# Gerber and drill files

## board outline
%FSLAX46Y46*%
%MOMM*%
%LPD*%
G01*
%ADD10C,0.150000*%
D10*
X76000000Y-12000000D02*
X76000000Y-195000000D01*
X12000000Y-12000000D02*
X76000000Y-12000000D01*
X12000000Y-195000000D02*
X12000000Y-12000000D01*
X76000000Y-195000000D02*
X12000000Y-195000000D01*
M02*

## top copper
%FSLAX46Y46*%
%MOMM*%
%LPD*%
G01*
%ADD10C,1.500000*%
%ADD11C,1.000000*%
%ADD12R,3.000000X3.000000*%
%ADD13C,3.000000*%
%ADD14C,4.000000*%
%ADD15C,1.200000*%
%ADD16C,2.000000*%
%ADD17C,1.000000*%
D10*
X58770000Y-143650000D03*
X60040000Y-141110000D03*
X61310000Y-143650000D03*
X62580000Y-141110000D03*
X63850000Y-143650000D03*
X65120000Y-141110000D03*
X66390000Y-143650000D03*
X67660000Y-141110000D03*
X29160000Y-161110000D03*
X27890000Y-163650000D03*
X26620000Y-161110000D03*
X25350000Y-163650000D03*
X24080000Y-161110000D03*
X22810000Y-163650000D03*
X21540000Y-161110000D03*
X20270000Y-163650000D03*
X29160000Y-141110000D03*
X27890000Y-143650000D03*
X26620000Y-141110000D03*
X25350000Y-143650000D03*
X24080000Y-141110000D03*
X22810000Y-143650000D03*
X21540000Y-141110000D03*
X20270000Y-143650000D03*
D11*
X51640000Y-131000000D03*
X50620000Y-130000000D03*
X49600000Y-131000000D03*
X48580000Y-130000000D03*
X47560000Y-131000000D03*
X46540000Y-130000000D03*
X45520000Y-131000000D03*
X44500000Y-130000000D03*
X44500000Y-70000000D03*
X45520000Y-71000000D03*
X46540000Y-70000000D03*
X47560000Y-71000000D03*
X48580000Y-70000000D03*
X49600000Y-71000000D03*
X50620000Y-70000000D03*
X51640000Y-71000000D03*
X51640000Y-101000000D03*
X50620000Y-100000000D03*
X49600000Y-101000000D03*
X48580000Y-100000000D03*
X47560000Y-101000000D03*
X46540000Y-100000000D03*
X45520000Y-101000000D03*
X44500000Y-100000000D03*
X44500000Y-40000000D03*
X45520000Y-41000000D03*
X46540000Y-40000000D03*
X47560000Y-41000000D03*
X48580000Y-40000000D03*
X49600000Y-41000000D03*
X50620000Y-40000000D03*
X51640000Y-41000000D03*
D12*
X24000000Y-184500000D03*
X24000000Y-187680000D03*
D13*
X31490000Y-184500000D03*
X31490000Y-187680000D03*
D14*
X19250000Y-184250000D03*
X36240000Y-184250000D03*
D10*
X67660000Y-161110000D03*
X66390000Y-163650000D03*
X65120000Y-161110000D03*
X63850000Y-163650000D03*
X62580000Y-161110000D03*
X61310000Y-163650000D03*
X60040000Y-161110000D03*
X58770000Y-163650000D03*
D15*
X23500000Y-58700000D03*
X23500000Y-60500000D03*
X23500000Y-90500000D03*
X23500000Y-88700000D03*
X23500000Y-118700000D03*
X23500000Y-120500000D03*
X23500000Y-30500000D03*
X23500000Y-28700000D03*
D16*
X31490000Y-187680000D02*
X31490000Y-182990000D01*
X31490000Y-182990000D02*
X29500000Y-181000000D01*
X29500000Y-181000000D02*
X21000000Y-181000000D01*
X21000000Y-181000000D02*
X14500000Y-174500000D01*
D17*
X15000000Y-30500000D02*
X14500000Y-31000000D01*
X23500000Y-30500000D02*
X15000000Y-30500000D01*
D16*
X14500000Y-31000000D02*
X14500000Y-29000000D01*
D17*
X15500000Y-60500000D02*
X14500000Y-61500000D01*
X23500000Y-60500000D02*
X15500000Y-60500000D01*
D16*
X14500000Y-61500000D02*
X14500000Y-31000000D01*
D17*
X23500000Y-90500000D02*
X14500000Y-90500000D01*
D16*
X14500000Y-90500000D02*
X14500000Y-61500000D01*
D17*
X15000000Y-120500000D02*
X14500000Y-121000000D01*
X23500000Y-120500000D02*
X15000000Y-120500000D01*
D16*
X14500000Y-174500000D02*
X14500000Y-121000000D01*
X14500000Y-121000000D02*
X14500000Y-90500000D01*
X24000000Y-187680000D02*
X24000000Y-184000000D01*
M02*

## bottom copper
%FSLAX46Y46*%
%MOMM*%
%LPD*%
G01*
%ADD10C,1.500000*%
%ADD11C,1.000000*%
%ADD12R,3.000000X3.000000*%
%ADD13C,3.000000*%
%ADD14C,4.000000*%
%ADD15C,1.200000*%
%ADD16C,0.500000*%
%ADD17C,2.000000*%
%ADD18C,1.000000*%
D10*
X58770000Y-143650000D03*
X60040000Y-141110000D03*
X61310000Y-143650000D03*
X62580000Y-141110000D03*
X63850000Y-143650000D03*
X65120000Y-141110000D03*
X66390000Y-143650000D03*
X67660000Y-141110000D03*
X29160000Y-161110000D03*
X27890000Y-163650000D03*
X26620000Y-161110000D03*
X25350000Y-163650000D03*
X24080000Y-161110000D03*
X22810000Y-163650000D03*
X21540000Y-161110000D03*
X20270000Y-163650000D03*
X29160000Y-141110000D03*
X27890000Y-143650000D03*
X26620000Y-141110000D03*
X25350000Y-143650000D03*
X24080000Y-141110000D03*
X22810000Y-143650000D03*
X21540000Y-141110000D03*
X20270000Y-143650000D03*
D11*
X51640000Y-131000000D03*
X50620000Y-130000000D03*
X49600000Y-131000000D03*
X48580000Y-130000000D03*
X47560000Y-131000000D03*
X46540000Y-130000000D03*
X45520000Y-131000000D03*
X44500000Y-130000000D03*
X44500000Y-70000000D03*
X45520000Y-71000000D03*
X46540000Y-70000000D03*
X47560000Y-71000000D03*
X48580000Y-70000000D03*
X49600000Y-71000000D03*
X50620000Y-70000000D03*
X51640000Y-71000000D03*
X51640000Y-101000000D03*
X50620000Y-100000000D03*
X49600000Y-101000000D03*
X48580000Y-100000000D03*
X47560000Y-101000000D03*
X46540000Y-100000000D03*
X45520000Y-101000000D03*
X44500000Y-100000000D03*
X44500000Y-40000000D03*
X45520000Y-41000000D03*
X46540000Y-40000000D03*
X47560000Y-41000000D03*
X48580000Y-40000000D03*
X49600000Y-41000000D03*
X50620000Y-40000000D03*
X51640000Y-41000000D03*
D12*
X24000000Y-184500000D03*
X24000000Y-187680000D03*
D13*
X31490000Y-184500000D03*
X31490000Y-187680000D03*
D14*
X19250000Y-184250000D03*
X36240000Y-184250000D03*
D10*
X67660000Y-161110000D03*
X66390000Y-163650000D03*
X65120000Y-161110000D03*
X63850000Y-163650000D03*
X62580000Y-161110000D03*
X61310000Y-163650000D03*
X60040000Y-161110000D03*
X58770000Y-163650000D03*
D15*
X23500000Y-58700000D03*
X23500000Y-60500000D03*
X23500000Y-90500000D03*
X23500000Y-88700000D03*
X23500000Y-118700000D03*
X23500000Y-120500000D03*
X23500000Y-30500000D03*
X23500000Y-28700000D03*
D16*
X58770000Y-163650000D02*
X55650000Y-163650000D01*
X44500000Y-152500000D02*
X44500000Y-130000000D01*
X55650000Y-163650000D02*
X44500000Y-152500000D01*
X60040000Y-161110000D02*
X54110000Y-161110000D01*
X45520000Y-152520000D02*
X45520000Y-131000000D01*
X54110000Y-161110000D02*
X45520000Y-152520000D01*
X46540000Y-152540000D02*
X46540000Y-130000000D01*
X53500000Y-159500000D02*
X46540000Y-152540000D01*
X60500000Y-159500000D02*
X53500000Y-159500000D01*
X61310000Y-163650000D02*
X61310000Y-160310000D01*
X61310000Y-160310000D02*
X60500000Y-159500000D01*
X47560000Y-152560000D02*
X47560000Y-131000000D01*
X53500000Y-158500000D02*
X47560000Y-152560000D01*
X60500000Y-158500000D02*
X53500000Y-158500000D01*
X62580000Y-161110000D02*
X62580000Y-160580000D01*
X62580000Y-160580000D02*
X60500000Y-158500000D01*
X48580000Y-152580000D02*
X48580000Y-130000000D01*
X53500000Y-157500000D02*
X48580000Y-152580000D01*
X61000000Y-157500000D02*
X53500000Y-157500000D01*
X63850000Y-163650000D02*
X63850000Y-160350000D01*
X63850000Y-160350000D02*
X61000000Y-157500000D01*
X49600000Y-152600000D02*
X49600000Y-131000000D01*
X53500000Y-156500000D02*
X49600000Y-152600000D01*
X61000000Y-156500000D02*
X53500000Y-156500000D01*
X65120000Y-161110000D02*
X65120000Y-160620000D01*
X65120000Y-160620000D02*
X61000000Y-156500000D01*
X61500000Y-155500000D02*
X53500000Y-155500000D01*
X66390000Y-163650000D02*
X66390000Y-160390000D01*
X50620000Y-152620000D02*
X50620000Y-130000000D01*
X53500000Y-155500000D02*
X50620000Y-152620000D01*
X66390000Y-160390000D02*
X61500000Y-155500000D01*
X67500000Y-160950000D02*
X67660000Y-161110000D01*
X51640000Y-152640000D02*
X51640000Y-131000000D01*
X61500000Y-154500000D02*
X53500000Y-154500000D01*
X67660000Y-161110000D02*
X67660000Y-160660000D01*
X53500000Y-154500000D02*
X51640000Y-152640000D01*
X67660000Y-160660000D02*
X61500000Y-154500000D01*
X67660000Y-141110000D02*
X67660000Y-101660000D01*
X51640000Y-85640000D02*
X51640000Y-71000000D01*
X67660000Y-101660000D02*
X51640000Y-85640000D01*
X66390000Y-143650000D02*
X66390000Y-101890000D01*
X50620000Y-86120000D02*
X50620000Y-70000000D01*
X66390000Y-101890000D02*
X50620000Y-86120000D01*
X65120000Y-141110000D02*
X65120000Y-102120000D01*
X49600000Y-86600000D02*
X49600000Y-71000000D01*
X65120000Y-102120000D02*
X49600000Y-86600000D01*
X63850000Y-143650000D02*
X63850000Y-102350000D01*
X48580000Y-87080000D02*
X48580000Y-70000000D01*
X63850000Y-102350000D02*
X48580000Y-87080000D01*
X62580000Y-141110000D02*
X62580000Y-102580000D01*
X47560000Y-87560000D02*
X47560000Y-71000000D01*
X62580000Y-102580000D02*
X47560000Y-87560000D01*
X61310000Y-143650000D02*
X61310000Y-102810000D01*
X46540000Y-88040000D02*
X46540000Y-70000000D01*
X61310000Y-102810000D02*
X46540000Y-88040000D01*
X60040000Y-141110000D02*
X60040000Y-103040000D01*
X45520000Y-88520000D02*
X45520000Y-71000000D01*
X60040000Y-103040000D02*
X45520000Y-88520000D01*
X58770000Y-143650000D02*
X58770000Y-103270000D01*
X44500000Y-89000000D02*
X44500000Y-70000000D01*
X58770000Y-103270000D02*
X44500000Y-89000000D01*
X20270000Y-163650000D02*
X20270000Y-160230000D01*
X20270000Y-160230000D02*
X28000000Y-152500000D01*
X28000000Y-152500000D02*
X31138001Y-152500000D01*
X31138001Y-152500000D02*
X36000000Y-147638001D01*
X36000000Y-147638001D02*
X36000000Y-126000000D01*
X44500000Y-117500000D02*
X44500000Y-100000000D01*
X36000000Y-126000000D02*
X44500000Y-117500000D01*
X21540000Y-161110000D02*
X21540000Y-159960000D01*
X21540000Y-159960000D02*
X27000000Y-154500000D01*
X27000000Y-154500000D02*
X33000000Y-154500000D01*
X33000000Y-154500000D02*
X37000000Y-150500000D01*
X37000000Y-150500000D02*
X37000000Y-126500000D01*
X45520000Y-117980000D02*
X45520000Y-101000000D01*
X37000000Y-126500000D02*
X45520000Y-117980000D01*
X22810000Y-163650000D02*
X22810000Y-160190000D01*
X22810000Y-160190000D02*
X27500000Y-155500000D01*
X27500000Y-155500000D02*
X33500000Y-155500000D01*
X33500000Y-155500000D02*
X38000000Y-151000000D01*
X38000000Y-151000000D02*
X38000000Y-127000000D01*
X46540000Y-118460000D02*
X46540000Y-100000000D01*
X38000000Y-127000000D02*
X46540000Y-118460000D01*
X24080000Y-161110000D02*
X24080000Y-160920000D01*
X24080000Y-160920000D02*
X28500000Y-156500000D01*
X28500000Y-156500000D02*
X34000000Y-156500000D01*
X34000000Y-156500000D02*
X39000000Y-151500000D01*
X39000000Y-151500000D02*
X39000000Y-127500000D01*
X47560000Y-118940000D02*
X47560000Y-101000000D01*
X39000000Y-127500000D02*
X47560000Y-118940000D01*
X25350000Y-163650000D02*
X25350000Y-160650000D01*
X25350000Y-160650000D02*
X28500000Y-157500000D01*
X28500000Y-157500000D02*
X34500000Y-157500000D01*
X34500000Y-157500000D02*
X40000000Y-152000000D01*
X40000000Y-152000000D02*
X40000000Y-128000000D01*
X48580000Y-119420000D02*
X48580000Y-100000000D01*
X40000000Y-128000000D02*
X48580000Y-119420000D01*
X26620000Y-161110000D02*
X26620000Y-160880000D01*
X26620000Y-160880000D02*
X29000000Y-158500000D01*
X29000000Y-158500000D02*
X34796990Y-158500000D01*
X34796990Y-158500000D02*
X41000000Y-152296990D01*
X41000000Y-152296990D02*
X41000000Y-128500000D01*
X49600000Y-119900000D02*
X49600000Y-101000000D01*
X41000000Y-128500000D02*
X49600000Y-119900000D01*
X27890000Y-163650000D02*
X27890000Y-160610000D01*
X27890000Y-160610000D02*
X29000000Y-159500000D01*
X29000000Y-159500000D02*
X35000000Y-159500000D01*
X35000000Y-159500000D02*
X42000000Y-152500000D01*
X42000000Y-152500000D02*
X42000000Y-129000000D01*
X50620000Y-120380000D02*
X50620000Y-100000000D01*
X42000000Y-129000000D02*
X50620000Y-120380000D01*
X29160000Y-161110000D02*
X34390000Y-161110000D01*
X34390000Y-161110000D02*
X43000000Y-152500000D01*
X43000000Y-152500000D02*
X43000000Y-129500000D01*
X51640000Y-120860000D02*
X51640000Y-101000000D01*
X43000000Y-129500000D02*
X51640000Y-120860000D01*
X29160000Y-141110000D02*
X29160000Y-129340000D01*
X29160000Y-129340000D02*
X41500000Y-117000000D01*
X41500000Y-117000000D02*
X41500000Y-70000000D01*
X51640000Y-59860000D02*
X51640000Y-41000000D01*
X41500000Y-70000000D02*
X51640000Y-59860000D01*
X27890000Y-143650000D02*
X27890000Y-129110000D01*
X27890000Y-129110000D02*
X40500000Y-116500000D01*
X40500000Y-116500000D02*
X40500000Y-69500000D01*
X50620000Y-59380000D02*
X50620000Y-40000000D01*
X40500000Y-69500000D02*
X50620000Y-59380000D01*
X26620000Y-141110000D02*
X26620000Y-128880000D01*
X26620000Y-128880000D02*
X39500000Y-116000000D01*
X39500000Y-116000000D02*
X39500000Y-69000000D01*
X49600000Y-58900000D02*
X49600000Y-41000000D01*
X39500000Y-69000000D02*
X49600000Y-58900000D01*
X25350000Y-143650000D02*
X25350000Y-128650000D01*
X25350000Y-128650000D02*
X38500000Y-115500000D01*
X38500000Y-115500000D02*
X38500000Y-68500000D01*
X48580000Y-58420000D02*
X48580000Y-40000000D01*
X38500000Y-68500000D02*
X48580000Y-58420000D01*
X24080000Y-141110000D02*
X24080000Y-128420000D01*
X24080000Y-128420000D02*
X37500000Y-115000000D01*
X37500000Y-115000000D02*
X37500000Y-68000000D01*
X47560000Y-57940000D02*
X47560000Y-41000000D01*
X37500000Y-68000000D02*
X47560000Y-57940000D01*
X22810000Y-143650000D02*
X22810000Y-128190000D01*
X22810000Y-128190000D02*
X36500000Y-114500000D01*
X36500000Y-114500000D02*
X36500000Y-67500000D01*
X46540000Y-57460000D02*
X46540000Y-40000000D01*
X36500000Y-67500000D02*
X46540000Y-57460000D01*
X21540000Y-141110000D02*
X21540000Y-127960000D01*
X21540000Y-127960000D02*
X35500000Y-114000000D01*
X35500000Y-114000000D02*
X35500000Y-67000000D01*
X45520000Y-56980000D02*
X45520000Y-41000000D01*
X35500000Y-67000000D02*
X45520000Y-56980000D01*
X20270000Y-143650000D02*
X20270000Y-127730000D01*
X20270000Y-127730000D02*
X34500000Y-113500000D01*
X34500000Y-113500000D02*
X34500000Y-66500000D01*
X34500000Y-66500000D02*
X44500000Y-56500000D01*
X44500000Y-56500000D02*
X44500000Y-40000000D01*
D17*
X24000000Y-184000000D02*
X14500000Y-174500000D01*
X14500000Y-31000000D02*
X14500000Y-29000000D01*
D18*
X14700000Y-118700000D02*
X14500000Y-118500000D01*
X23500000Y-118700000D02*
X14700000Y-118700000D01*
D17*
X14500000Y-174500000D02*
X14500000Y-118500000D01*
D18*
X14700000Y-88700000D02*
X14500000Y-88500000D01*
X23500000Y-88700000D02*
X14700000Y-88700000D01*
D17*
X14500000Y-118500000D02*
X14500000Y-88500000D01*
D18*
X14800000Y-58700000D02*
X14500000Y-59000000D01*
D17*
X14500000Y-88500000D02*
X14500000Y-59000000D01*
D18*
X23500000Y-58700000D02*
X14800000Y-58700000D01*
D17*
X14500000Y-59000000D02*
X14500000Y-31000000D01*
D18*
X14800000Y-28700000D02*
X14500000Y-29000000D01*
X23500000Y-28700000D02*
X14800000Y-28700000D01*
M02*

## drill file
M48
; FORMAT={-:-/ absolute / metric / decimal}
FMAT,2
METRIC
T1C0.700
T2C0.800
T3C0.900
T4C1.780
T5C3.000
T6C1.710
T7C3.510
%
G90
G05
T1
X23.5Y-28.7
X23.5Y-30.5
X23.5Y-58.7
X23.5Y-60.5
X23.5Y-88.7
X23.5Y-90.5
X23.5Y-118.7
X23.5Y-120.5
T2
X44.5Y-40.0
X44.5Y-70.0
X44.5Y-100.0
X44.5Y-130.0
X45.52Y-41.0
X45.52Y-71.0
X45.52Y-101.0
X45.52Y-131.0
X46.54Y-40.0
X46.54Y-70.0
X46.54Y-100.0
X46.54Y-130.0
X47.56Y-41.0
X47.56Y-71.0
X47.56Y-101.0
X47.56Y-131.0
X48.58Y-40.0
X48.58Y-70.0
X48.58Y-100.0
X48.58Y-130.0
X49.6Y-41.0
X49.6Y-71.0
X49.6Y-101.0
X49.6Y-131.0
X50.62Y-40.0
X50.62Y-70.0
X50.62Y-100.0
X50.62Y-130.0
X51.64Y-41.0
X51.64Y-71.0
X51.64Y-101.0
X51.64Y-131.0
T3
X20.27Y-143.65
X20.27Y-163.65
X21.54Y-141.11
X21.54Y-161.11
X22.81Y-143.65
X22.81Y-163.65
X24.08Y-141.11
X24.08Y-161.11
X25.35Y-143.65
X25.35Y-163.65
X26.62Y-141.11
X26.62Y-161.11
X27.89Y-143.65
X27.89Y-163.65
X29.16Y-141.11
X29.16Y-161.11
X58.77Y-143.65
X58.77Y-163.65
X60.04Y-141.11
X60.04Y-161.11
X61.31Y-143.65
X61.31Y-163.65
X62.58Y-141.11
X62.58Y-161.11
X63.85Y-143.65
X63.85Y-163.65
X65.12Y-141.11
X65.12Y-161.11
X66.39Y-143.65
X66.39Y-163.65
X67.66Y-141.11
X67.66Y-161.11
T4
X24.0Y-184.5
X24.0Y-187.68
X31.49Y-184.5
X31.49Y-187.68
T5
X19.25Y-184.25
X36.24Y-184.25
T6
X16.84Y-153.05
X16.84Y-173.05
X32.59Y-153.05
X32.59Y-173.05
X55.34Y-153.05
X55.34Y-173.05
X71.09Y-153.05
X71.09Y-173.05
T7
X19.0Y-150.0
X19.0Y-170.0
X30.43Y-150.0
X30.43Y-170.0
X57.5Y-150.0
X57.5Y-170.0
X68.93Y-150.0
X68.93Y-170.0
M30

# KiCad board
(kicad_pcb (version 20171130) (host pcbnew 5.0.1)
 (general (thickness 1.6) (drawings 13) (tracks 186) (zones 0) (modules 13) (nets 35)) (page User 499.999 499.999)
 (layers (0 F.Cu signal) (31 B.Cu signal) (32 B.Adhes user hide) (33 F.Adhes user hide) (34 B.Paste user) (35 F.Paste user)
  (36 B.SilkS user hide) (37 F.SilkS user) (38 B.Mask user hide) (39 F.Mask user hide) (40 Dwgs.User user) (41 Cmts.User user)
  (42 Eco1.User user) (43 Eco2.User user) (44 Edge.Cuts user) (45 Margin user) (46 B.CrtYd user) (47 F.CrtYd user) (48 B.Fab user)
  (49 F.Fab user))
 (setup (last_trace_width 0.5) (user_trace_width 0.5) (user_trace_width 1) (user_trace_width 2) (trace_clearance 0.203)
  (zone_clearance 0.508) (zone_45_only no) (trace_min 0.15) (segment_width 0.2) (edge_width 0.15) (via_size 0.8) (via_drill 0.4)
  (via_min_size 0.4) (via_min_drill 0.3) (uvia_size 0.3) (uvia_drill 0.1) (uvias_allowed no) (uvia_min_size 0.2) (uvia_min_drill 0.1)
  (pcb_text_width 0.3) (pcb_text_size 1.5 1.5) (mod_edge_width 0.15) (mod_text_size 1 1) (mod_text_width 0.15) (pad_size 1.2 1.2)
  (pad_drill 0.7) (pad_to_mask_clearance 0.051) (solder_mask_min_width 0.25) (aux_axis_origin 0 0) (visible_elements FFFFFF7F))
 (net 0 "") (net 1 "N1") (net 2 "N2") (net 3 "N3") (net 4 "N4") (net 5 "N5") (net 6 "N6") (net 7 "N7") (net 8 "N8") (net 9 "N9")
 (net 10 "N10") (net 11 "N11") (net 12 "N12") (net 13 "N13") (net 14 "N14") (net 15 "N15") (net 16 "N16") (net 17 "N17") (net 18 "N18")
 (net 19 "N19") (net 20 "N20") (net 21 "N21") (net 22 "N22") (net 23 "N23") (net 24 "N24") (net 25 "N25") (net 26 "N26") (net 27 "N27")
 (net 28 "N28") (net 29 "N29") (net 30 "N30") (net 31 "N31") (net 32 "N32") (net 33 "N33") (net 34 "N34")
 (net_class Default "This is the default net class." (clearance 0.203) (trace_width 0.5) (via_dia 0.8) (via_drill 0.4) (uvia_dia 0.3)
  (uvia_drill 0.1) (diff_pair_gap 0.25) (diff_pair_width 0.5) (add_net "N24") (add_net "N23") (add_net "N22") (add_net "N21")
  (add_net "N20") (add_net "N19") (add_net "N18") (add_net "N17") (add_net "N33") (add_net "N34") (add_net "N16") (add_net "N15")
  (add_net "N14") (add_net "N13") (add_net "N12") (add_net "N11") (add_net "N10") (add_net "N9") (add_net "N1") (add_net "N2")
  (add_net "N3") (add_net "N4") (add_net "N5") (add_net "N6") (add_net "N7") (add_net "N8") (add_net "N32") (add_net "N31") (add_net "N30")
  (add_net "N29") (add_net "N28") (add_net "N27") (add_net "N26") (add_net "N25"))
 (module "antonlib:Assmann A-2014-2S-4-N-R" (layer F.Cu) (at 57.5 150 180)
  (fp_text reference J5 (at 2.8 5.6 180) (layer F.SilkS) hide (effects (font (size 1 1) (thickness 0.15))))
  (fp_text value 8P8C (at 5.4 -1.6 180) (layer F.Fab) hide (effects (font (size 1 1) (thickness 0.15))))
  (pad "" np_thru_hole circle (at 0 0 180) (size 3.51 3.51) (drill 3.51) (layers *.Cu *.Mask))
  (pad "" np_thru_hole circle (at -11.43 0 180) (size 3.51 3.51) (drill 3.51) (layers *.Cu *.Mask))
  (pad "" np_thru_hole circle (at 2.16 -3.05 180) (size 1.71 1.71) (drill 1.71) (layers *.Cu *.Mask))
  (pad "" np_thru_hole circle (at -13.59 -3.05 180) (size 1.71 1.71) (drill 1.71) (layers *.Cu *.Mask))
  (pad 1 thru_hole circle (at -1.27 6.35 180) (size 1.5 1.5) (drill 0.9) (layers *.Cu *.Mask) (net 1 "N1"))
  (pad 2 thru_hole circle (at -2.54 8.89 180) (size 1.5 1.5) (drill 0.9) (layers *.Cu *.Mask) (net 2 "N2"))
  (pad 3 thru_hole circle (at -3.81 6.35 180) (size 1.5 1.5) (drill 0.9) (layers *.Cu *.Mask) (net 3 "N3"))
  (pad 4 thru_hole circle (at -5.08 8.89 180) (size 1.5 1.5) (drill 0.9) (layers *.Cu *.Mask) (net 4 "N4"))
  (pad 5 thru_hole circle (at -6.35 6.35 180) (size 1.5 1.5) (drill 0.9) (layers *.Cu *.Mask) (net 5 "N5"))
  (pad 6 thru_hole circle (at -7.62 8.89 180) (size 1.5 1.5) (drill 0.9) (layers *.Cu *.Mask) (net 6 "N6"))
  (pad 7 thru_hole circle (at -8.89 6.35 180) (size 1.5 1.5) (drill 0.9) (layers *.Cu *.Mask) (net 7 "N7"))
  (pad 8 thru_hole circle (at -10.16 8.89 180) (size 1.5 1.5) (drill 0.9) (layers *.Cu *.Mask) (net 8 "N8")))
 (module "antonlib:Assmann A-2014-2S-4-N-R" (layer F.Cu) (at 19 170 180)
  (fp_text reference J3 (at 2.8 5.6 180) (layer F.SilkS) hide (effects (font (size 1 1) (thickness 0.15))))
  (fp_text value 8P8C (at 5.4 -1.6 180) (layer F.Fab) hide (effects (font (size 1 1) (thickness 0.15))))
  (pad 8 thru_hole circle (at -10.16 8.89 180) (size 1.5 1.5) (drill 0.9) (layers *.Cu *.Mask) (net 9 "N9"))
  (pad 7 thru_hole circle (at -8.89 6.35 180) (size 1.5 1.5) (drill 0.9) (layers *.Cu *.Mask) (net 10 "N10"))
  (pad 6 thru_hole circle (at -7.62 8.89 180) (size 1.5 1.5) (drill 0.9) (layers *.Cu *.Mask) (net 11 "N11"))
  (pad 5 thru_hole circle (at -6.35 6.35 180) (size 1.5 1.5) (drill 0.9) (layers *.Cu *.Mask) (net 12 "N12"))
  (pad 4 thru_hole circle (at -5.08 8.89 180) (size 1.5 1.5) (drill 0.9) (layers *.Cu *.Mask) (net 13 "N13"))
  (pad 3 thru_hole circle (at -3.81 6.35 180) (size 1.5 1.5) (drill 0.9) (layers *.Cu *.Mask) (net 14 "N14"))
  (pad 2 thru_hole circle (at -2.54 8.89 180) (size 1.5 1.5) (drill 0.9) (layers *.Cu *.Mask) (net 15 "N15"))
  (pad 1 thru_hole circle (at -1.27 6.35 180) (size 1.5 1.5) (drill 0.9) (layers *.Cu *.Mask) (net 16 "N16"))
  (pad "" np_thru_hole circle (at -13.59 -3.05 180) (size 1.71 1.71) (drill 1.71) (layers *.Cu *.Mask))
  (pad "" np_thru_hole circle (at 2.16 -3.05 180) (size 1.71 1.71) (drill 1.71) (layers *.Cu *.Mask))
  (pad "" np_thru_hole circle (at -11.43 0 180) (size 3.51 3.51) (drill 3.51) (layers *.Cu *.Mask))
  (pad "" np_thru_hole circle (at 0 0 180) (size 3.51 3.51) (drill 3.51) (layers *.Cu *.Mask)))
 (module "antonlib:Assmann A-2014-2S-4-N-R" (layer F.Cu) (at 19 150 180)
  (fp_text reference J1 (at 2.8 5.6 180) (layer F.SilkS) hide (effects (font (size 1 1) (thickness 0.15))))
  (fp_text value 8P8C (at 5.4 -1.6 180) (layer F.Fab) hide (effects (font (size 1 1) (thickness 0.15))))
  (pad 8 thru_hole circle (at -10.16 8.89 180) (size 1.5 1.5) (drill 0.9) (layers *.Cu *.Mask) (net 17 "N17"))
  (pad 7 thru_hole circle (at -8.89 6.35 180) (size 1.5 1.5) (drill 0.9) (layers *.Cu *.Mask) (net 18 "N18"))
  (pad 6 thru_hole circle (at -7.62 8.89 180) (size 1.5 1.5) (drill 0.9) (layers *.Cu *.Mask) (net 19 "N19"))
  (pad 5 thru_hole circle (at -6.35 6.35 180) (size 1.5 1.5) (drill 0.9) (layers *.Cu *.Mask) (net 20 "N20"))
  (pad 4 thru_hole circle (at -5.08 8.89 180) (size 1.5 1.5) (drill 0.9) (layers *.Cu *.Mask) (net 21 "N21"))
  (pad 3 thru_hole circle (at -3.81 6.35 180) (size 1.5 1.5) (drill 0.9) (layers *.Cu *.Mask) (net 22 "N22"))
  (pad 2 thru_hole circle (at -2.54 8.89 180) (size 1.5 1.5) (drill 0.9) (layers *.Cu *.Mask) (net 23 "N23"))
  (pad 1 thru_hole circle (at -1.27 6.35 180) (size 1.5 1.5) (drill 0.9) (layers *.Cu *.Mask) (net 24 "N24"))
  (pad "" np_thru_hole circle (at -13.59 -3.05 180) (size 1.71 1.71) (drill 1.71) (layers *.Cu *.Mask))
  (pad "" np_thru_hole circle (at 2.16 -3.05 180) (size 1.71 1.71) (drill 1.71) (layers *.Cu *.Mask))
  (pad "" np_thru_hole circle (at -11.43 0 180) (size 3.51 3.51) (drill 3.51) (layers *.Cu *.Mask))
  (pad "" np_thru_hole circle (at 0 0 180) (size 3.51 3.51) (drill 3.51) (layers *.Cu *.Mask)))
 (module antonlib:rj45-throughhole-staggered (layer F.Cu) (at 44.5 130)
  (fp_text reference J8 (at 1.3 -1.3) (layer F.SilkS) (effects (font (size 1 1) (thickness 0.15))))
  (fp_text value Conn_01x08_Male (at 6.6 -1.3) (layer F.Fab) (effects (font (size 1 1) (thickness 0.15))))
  (pad 8 thru_hole circle (at 7.14 1) (size 1 1) (drill 0.8) (layers *.Cu *.Mask) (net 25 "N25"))
  (pad 7 thru_hole circle (at 6.12 0) (size 1 1) (drill 0.8) (layers *.Cu *.Mask) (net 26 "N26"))
  (pad 6 thru_hole circle (at 5.1 1) (size 1 1) (drill 0.8) (layers *.Cu *.Mask) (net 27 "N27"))
  (pad 5 thru_hole circle (at 4.08 0) (size 1 1) (drill 0.8) (layers *.Cu *.Mask) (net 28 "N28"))
  (pad 4 thru_hole circle (at 3.06 1) (size 1 1) (drill 0.8) (layers *.Cu *.Mask) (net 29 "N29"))
  (pad 3 thru_hole circle (at 2.04 0) (size 1 1) (drill 0.8) (layers *.Cu *.Mask) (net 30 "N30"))
  (pad 2 thru_hole circle (at 1.02 1) (size 1 1) (drill 0.8) (layers *.Cu *.Mask) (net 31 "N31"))
  (pad 1 thru_hole circle (at 0 0) (size 1 1) (drill 0.8) (layers *.Cu *.Mask) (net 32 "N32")))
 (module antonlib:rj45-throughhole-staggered (layer F.Cu) (at 44.5 70)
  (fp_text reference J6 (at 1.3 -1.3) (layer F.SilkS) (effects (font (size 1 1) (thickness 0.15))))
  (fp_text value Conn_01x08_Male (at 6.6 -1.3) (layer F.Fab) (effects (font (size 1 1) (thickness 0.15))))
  (pad 1 thru_hole circle (at 0 0) (size 1 1) (drill 0.8) (layers *.Cu *.Mask) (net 1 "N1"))
  (pad 2 thru_hole circle (at 1.02 1) (size 1 1) (drill 0.8) (layers *.Cu *.Mask) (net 2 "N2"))
  (pad 3 thru_hole circle (at 2.04 0) (size 1 1) (drill 0.8) (layers *.Cu *.Mask) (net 3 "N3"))
  (pad 4 thru_hole circle (at 3.06 1) (size 1 1) (drill 0.8) (layers *.Cu *.Mask) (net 4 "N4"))
  (pad 5 thru_hole circle (at 4.08 0) (size 1 1) (drill 0.8) (layers *.Cu *.Mask) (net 5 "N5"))
  (pad 6 thru_hole circle (at 5.1 1) (size 1 1) (drill 0.8) (layers *.Cu *.Mask) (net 6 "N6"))
  (pad 7 thru_hole circle (at 6.12 0) (size 1 1) (drill 0.8) (layers *.Cu *.Mask) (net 7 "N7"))
  (pad 8 thru_hole circle (at 7.14 1) (size 1 1) (drill 0.8) (layers *.Cu *.Mask) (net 8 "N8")))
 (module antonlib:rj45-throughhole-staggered (layer F.Cu) (at 44.5 100)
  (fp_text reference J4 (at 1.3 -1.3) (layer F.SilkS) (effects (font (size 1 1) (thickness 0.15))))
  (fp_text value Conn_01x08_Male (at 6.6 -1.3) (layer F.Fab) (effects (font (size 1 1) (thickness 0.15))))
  (pad 8 thru_hole circle (at 7.14 1) (size 1 1) (drill 0.8) (layers *.Cu *.Mask) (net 9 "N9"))
  (pad 7 thru_hole circle (at 6.12 0) (size 1 1) (drill 0.8) (layers *.Cu *.Mask) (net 10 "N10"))
  (pad 6 thru_hole circle (at 5.1 1) (size 1 1) (drill 0.8) (layers *.Cu *.Mask) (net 11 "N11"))
  (pad 5 thru_hole circle (at 4.08 0) (size 1 1) (drill 0.8) (layers *.Cu *.Mask) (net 12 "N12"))
  (pad 4 thru_hole circle (at 3.06 1) (size 1 1) (drill 0.8) (layers *.Cu *.Mask) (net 13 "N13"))
  (pad 3 thru_hole circle (at 2.04 0) (size 1 1) (drill 0.8) (layers *.Cu *.Mask) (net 14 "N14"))
  (pad 2 thru_hole circle (at 1.02 1) (size 1 1) (drill 0.8) (layers *.Cu *.Mask) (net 15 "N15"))
  (pad 1 thru_hole circle (at 0 0) (size 1 1) (drill 0.8) (layers *.Cu *.Mask) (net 16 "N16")))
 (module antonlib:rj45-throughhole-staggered (layer F.Cu) (at 44.5 40)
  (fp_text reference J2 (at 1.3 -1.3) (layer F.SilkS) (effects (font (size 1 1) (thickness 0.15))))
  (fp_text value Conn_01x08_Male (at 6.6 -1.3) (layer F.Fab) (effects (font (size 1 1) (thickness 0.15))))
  (pad 1 thru_hole circle (at 0 0) (size 1 1) (drill 0.8) (layers *.Cu *.Mask) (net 24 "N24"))
  (pad 2 thru_hole circle (at 1.02 1) (size 1 1) (drill 0.8) (layers *.Cu *.Mask) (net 23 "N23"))
  (pad 3 thru_hole circle (at 2.04 0) (size 1 1) (drill 0.8) (layers *.Cu *.Mask) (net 22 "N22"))
  (pad 4 thru_hole circle (at 3.06 1) (size 1 1) (drill 0.8) (layers *.Cu *.Mask) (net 21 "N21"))
  (pad 5 thru_hole circle (at 4.08 0) (size 1 1) (drill 0.8) (layers *.Cu *.Mask) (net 20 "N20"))
  (pad 6 thru_hole circle (at 5.1 1) (size 1 1) (drill 0.8) (layers *.Cu *.Mask) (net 19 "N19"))
  (pad 7 thru_hole circle (at 6.12 0) (size 1 1) (drill 0.8) (layers *.Cu *.Mask) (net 18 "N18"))
  (pad 8 thru_hole circle (at 7.14 1) (size 1 1) (drill 0.8) (layers *.Cu *.Mask) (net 17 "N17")))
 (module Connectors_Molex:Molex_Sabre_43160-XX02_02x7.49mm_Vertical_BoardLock (layer F.Cu) (at 24 184.5)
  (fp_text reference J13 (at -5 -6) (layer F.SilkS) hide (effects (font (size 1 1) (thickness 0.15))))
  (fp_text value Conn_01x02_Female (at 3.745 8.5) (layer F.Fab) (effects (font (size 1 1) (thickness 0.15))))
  (pad 1 thru_hole rect (at 0 0) (size 3 3) (drill 1.78) (layers *.Cu *.Mask) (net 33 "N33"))
  (pad 1 thru_hole rect (at 0 3.18) (size 3 3) (drill 1.78) (layers *.Cu *.Mask) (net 33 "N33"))
  (pad 2 thru_hole circle (at 7.49 0) (size 3 3) (drill 1.78) (layers *.Cu *.Mask) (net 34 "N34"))
  (pad 2 thru_hole circle (at 7.49 3.18) (size 3 3) (drill 1.78) (layers *.Cu *.Mask) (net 34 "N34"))
  (pad "" thru_hole circle (at -4.75 -0.25) (size 4 4) (drill 3) (layers *.Cu *.Mask))
  (pad "" thru_hole circle (at 12.24 -0.25) (size 4 4) (drill 3) (layers *.Cu *.Mask)))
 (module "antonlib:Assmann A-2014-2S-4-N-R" (layer F.Cu) (at 57.5 170 180)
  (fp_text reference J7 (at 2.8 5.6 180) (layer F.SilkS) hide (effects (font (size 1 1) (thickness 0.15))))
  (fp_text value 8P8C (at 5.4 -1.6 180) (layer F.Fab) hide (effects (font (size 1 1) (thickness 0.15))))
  (pad 8 thru_hole circle (at -10.16 8.89 180) (size 1.5 1.5) (drill 0.9) (layers *.Cu *.Mask) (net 25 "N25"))
  (pad 7 thru_hole circle (at -8.89 6.35 180) (size 1.5 1.5) (drill 0.9) (layers *.Cu *.Mask) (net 26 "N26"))
  (pad 6 thru_hole circle (at -7.62 8.89 180) (size 1.5 1.5) (drill 0.9) (layers *.Cu *.Mask) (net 27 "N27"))
  (pad 5 thru_hole circle (at -6.35 6.35 180) (size 1.5 1.5) (drill 0.9) (layers *.Cu *.Mask) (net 28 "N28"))
  (pad 4 thru_hole circle (at -5.08 8.89 180) (size 1.5 1.5) (drill 0.9) (layers *.Cu *.Mask) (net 29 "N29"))
  (pad 3 thru_hole circle (at -3.81 6.35 180) (size 1.5 1.5) (drill 0.9) (layers *.Cu *.Mask) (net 30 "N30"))
  (pad 2 thru_hole circle (at -2.54 8.89 180) (size 1.5 1.5) (drill 0.9) (layers *.Cu *.Mask) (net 31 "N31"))
  (pad 1 thru_hole circle (at -1.27 6.35 180) (size 1.5 1.5) (drill 0.9) (layers *.Cu *.Mask) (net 32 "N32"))
  (pad "" np_thru_hole circle (at -13.59 -3.05 180) (size 1.71 1.71) (drill 1.71) (layers *.Cu *.Mask))
  (pad "" np_thru_hole circle (at 2.16 -3.05 180) (size 1.71 1.71) (drill 1.71) (layers *.Cu *.Mask))
  (pad "" np_thru_hole circle (at -11.43 0 180) (size 3.51 3.51) (drill 3.51) (layers *.Cu *.Mask))
  (pad "" np_thru_hole circle (at 0 0 180) (size 3.51 3.51) (drill 3.51) (layers *.Cu *.Mask)))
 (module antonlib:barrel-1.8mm (layer F.Cu) (at 23.5 60.5 90)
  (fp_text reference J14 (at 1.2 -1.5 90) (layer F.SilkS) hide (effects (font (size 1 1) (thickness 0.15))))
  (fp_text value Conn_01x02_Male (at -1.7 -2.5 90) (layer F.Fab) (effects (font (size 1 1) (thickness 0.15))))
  (pad 2 thru_hole circle (at 1.8 0 90) (size 1.2 1.2) (drill 0.7) (layers *.Cu *.Mask) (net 33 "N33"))
  (pad 1 thru_hole circle (at 0 0 90) (size 1.2 1.2) (drill 0.7) (layers *.Cu *.Mask) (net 34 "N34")))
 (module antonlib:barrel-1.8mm (layer F.Cu) (at 23.5 90.5 90)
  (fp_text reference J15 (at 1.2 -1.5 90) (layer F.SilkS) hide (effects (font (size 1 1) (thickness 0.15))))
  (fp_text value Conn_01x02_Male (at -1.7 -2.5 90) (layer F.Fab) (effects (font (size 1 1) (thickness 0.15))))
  (pad 1 thru_hole circle (at 0 0 90) (size 1.2 1.2) (drill 0.7) (layers *.Cu *.Mask) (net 34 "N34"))
  (pad 2 thru_hole circle (at 1.8 0 90) (size 1.2 1.2) (drill 0.7) (layers *.Cu *.Mask) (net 33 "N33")))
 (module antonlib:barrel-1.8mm (layer F.Cu) (at 23.5 120.5 90)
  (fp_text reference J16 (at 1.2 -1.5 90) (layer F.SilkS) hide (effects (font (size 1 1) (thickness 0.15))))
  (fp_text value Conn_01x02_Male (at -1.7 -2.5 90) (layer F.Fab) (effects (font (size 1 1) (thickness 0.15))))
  (pad 2 thru_hole circle (at 1.8 0 90) (size 1.2 1.2) (drill 0.7) (layers *.Cu *.Mask) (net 33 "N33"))
  (pad 1 thru_hole circle (at 0 0 90) (size 1.2 1.2) (drill 0.7) (layers *.Cu *.Mask) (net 34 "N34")))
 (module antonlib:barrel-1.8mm (layer F.Cu) (at 23.5 30.5 90)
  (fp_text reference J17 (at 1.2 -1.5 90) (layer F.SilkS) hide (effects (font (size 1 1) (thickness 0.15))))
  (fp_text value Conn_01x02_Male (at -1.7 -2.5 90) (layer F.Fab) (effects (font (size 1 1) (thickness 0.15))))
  (pad 1 thru_hole circle (at 0 0 90) (size 1.2 1.2) (drill 0.7) (layers *.Cu *.Mask) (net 34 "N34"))
  (pad 2 thru_hole circle (at 1.8 0 90) (size 1.2 1.2) (drill 0.7) (layers *.Cu *.Mask) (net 33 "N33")))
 (gr_line (start 76 12) (end 76 195) (layer Edge.Cuts) (width 0.15))
 (gr_line (start 12 12) (end 76 12) (layer Edge.Cuts) (width 0.15))
 (gr_line (start 12 195) (end 12 12) (layer Edge.Cuts) (width 0.15))
 (gr_line (start 76 195) (end 12 195) (layer Edge.Cuts) (width 0.15))
 (segment (start 58.77 163.65) (end 55.65 163.65) (width 0.5) (layer B.Cu) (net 32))
 (segment (start 44.5 152.5) (end 44.5 130) (width 0.5) (layer B.Cu) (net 32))
 (segment (start 55.65 163.65) (end 44.5 152.5) (width 0.5) (layer B.Cu) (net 32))
 (segment (start 60.04 161.11) (end 54.11 161.11) (width 0.5) (layer B.Cu) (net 31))
 (segment (start 45.52 152.52) (end 45.52 131) (width 0.5) (layer B.Cu) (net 31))
 (segment (start 54.11 161.11) (end 45.52 152.52) (width 0.5) (layer B.Cu) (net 31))
 (segment (start 46.54 152.54) (end 46.54 130) (width 0.5) (layer B.Cu) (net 30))
 (segment (start 53.5 159.5) (end 46.54 152.54) (width 0.5) (layer B.Cu) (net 30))
 (segment (start 60.5 159.5) (end 53.5 159.5) (width 0.5) (layer B.Cu) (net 30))
 (segment (start 61.31 163.65) (end 61.31 160.31) (width 0.5) (layer B.Cu) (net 30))
 (segment (start 61.31 160.31) (end 60.5 159.5) (width 0.5) (layer B.Cu) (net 30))
 (segment (start 47.56 152.56) (end 47.56 131) (width 0.5) (layer B.Cu) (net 29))
 (segment (start 53.5 158.5) (end 47.56 152.56) (width 0.5) (layer B.Cu) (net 29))
 (segment (start 60.5 158.5) (end 53.5 158.5) (width 0.5) (layer B.Cu) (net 29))
 (segment (start 62.58 161.11) (end 62.58 160.58) (width 0.5) (layer B.Cu) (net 29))
 (segment (start 62.58 160.58) (end 60.5 158.5) (width 0.5) (layer B.Cu) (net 29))
 (segment (start 48.58 152.58) (end 48.58 130) (width 0.5) (layer B.Cu) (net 28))
 (segment (start 53.5 157.5) (end 48.58 152.58) (width 0.5) (layer B.Cu) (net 28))
 (segment (start 61 157.5) (end 53.5 157.5) (width 0.5) (layer B.Cu) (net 28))
 (segment (start 63.85 163.65) (end 63.85 160.35) (width 0.5) (layer B.Cu) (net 28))
 (segment (start 63.85 160.35) (end 61 157.5) (width 0.5) (layer B.Cu) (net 28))
 (segment (start 49.6 152.6) (end 49.6 131) (width 0.5) (layer B.Cu) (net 27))
 (segment (start 53.5 156.5) (end 49.6 152.6) (width 0.5) (layer B.Cu) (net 27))
 (segment (start 61 156.5) (end 53.5 156.5) (width 0.5) (layer B.Cu) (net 27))
 (segment (start 65.12 161.11) (end 65.12 160.62) (width 0.5) (layer B.Cu) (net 27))
 (segment (start 65.12 160.62) (end 61 156.5) (width 0.5) (layer B.Cu) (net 27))
 (segment (start 61.5 155.5) (end 53.5 155.5) (width 0.5) (layer B.Cu) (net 26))
 (segment (start 66.39 163.65) (end 66.39 160.39) (width 0.5) (layer B.Cu) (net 26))
 (segment (start 50.62 152.62) (end 50.62 130) (width 0.5) (layer B.Cu) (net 26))
 (segment (start 53.5 155.5) (end 50.62 152.62) (width 0.5) (layer B.Cu) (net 26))
 (segment (start 66.39 160.39) (end 61.5 155.5) (width 0.5) (layer B.Cu) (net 26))
 (segment (start 67.5 160.95) (end 67.66 161.11) (width 0.5) (layer B.Cu) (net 25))
 (segment (start 51.64 152.64) (end 51.64 131) (width 0.5) (layer B.Cu) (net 25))
 (segment (start 61.5 154.5) (end 53.5 154.5) (width 0.5) (layer B.Cu) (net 25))
 (segment (start 67.66 161.11) (end 67.66 160.66) (width 0.5) (layer B.Cu) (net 25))
 (segment (start 53.5 154.5) (end 51.64 152.64) (width 0.5) (layer B.Cu) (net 25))
 (segment (start 67.66 160.66) (end 61.5 154.5) (width 0.5) (layer B.Cu) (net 25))
 (segment (start 67.66 141.11) (end 67.66 101.66) (width 0.5) (layer B.Cu) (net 8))
 (segment (start 51.64 85.64) (end 51.64 71) (width 0.5) (layer B.Cu) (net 8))
 (segment (start 67.66 101.66) (end 51.64 85.64) (width 0.5) (layer B.Cu) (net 8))
 (segment (start 66.39 143.65) (end 66.39 101.89) (width 0.5) (layer B.Cu) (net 7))
 (segment (start 50.62 86.12) (end 50.62 70) (width 0.5) (layer B.Cu) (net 7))
 (segment (start 66.39 101.89) (end 50.62 86.12) (width 0.5) (layer B.Cu) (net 7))
 (segment (start 65.12 141.11) (end 65.12 102.12) (width 0.5) (layer B.Cu) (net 6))
 (segment (start 49.6 86.6) (end 49.6 71) (width 0.5) (layer B.Cu) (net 6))
 (segment (start 65.12 102.12) (end 49.6 86.6) (width 0.5) (layer B.Cu) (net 6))
 (segment (start 63.85 143.65) (end 63.85 102.35) (width 0.5) (layer B.Cu) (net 5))
 (segment (start 48.58 87.08) (end 48.58 70) (width 0.5) (layer B.Cu) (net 5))
 (segment (start 63.85 102.35) (end 48.58 87.08) (width 0.5) (layer B.Cu) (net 5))
 (segment (start 62.58 141.11) (end 62.58 102.58) (width 0.5) (layer B.Cu) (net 4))
 (segment (start 47.56 87.56) (end 47.56 71) (width 0.5) (layer B.Cu) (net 4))
 (segment (start 62.58 102.58) (end 47.56 87.56) (width 0.5) (layer B.Cu) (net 4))
 (segment (start 61.31 143.65) (end 61.31 102.81) (width 0.5) (layer B.Cu) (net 3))
 (segment (start 46.54 88.04) (end 46.54 70) (width 0.5) (layer B.Cu) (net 3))
 (segment (start 61.31 102.81) (end 46.54 88.04) (width 0.5) (layer B.Cu) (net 3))
 (segment (start 60.04 141.11) (end 60.04 103.04) (width 0.5) (layer B.Cu) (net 2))
 (segment (start 45.52 88.52) (end 45.52 71) (width 0.5) (layer B.Cu) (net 2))
 (segment (start 60.04 103.04) (end 45.52 88.52) (width 0.5) (layer B.Cu) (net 2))
 (segment (start 58.77 143.65) (end 58.77 103.27) (width 0.5) (layer B.Cu) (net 1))
 (segment (start 44.5 89) (end 44.5 70) (width 0.5) (layer B.Cu) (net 1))
 (segment (start 58.77 103.27) (end 44.5 89) (width 0.5) (layer B.Cu) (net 1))
 (segment (start 20.27 163.65) (end 20.27 160.23) (width 0.5) (layer B.Cu) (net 16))
 (segment (start 20.27 160.23) (end 28 152.5) (width 0.5) (layer B.Cu) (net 16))
 (segment (start 28 152.5) (end 31.138001 152.5) (width 0.5) (layer B.Cu) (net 16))
 (segment (start 31.138001 152.5) (end 36 147.638001) (width 0.5) (layer B.Cu) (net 16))
 (segment (start 36 147.638001) (end 36 126) (width 0.5) (layer B.Cu) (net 16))
 (segment (start 44.5 117.5) (end 44.5 100) (width 0.5) (layer B.Cu) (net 16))
 (segment (start 36 126) (end 44.5 117.5) (width 0.5) (layer B.Cu) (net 16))
 (segment (start 21.54 161.11) (end 21.54 159.96) (width 0.5) (layer B.Cu) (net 15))
 (segment (start 21.54 159.96) (end 27 154.5) (width 0.5) (layer B.Cu) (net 15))
 (segment (start 27 154.5) (end 33 154.5) (width 0.5) (layer B.Cu) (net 15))
 (segment (start 33 154.5) (end 37 150.5) (width 0.5) (layer B.Cu) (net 15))
 (segment (start 37 150.5) (end 37 126.5) (width 0.5) (layer B.Cu) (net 15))
 (segment (start 45.52 117.98) (end 45.52 101) (width 0.5) (layer B.Cu) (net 15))
 (segment (start 37 126.5) (end 45.52 117.98) (width 0.5) (layer B.Cu) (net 15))
 (segment (start 22.81 163.65) (end 22.81 160.19) (width 0.5) (layer B.Cu) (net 14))
 (segment (start 22.81 160.19) (end 27.5 155.5) (width 0.5) (layer B.Cu) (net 14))
 (segment (start 27.5 155.5) (end 33.5 155.5) (width 0.5) (layer B.Cu) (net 14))
 (segment (start 33.5 155.5) (end 38 151) (width 0.5) (layer B.Cu) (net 14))
 (segment (start 38 151) (end 38 127) (width 0.5) (layer B.Cu) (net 14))
 (segment (start 46.54 118.46) (end 46.54 100) (width 0.5) (layer B.Cu) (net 14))
 (segment (start 38 127) (end 46.54 118.46) (width 0.5) (layer B.Cu) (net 14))
 (segment (start 24.08 161.11) (end 24.08 160.92) (width 0.5) (layer B.Cu) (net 13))
 (segment (start 24.08 160.92) (end 28.5 156.5) (width 0.5) (layer B.Cu) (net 13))
 (segment (start 28.5 156.5) (end 34 156.5) (width 0.5) (layer B.Cu) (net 13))
 (segment (start 34 156.5) (end 39 151.5) (width 0.5) (layer B.Cu) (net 13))
 (segment (start 39 151.5) (end 39 127.5) (width 0.5) (layer B.Cu) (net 13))
 (segment (start 47.56 118.94) (end 47.56 101) (width 0.5) (layer B.Cu) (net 13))
 (segment (start 39 127.5) (end 47.56 118.94) (width 0.5) (layer B.Cu) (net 13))
 (segment (start 25.35 163.65) (end 25.35 160.65) (width 0.5) (layer B.Cu) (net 12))
 (segment (start 25.35 160.65) (end 28.5 157.5) (width 0.5) (layer B.Cu) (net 12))
 (segment (start 28.5 157.5) (end 34.5 157.5) (width 0.5) (layer B.Cu) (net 12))
 (segment (start 34.5 157.5) (end 40 152) (width 0.5) (layer B.Cu) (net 12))
 (segment (start 40 152) (end 40 128) (width 0.5) (layer B.Cu) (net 12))
 (segment (start 48.58 119.42) (end 48.58 100) (width 0.5) (layer B.Cu) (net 12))
 (segment (start 40 128) (end 48.58 119.42) (width 0.5) (layer B.Cu) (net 12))
 (segment (start 26.62 161.11) (end 26.62 160.88) (width 0.5) (layer B.Cu) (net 11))
 (segment (start 26.62 160.88) (end 29 158.5) (width 0.5) (layer B.Cu) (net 11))
 (segment (start 29 158.5) (end 34.79699 158.5) (width 0.5) (layer B.Cu) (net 11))
 (segment (start 34.79699 158.5) (end 41 152.29699) (width 0.5) (layer B.Cu) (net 11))
 (segment (start 41 152.29699) (end 41 128.5) (width 0.5) (layer B.Cu) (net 11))
 (segment (start 49.6 119.9) (end 49.6 101) (width 0.5) (layer B.Cu) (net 11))
 (segment (start 41 128.5) (end 49.6 119.9) (width 0.5) (layer B.Cu) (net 11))
 (segment (start 27.89 163.65) (end 27.89 160.61) (width 0.5) (layer B.Cu) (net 10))
 (segment (start 27.89 160.61) (end 29 159.5) (width 0.5) (layer B.Cu) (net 10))
 (segment (start 29 159.5) (end 35 159.5) (width 0.5) (layer B.Cu) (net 10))
 (segment (start 35 159.5) (end 42 152.5) (width 0.5) (layer B.Cu) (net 10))
 (segment (start 42 152.5) (end 42 129) (width 0.5) (layer B.Cu) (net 10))
 (segment (start 50.62 120.38) (end 50.62 100) (width 0.5) (layer B.Cu) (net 10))
 (segment (start 42 129) (end 50.62 120.38) (width 0.5) (layer B.Cu) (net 10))
 (segment (start 29.16 161.11) (end 34.39 161.11) (width 0.5) (layer B.Cu) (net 9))
 (segment (start 34.39 161.11) (end 43 152.5) (width 0.5) (layer B.Cu) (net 9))
 (segment (start 43 152.5) (end 43 129.5) (width 0.5) (layer B.Cu) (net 9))
 (segment (start 51.64 120.86) (end 51.64 101) (width 0.5) (layer B.Cu) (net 9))
 (segment (start 43 129.5) (end 51.64 120.86) (width 0.5) (layer B.Cu) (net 9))
 (segment (start 29.16 141.11) (end 29.16 129.34) (width 0.5) (layer B.Cu) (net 17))
 (segment (start 29.16 129.34) (end 41.5 117) (width 0.5) (layer B.Cu) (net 17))
 (segment (start 41.5 117) (end 41.5 70) (width 0.5) (layer B.Cu) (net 17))
 (segment (start 51.64 59.86) (end 51.64 41) (width 0.5) (layer B.Cu) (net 17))
 (segment (start 41.5 70) (end 51.64 59.86) (width 0.5) (layer B.Cu) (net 17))
 (segment (start 27.89 143.65) (end 27.89 129.11) (width 0.5) (layer B.Cu) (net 18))
 (segment (start 27.89 129.11) (end 40.5 116.5) (width 0.5) (layer B.Cu) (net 18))
 (segment (start 40.5 116.5) (end 40.5 69.5) (width 0.5) (layer B.Cu) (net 18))
 (segment (start 50.62 59.38) (end 50.62 40) (width 0.5) (layer B.Cu) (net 18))
 (segment (start 40.5 69.5) (end 50.62 59.38) (width 0.5) (layer B.Cu) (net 18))
 (segment (start 26.62 141.11) (end 26.62 128.88) (width 0.5) (layer B.Cu) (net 19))
 (segment (start 26.62 128.88) (end 39.5 116) (width 0.5) (layer B.Cu) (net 19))
 (segment (start 39.5 116) (end 39.5 69) (width 0.5) (layer B.Cu) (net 19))
 (segment (start 49.6 58.9) (end 49.6 41) (width 0.5) (layer B.Cu) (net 19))
 (segment (start 39.5 69) (end 49.6 58.9) (width 0.5) (layer B.Cu) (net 19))
 (segment (start 25.35 143.65) (end 25.35 128.65) (width 0.5) (layer B.Cu) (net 20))
 (segment (start 25.35 128.65) (end 38.5 115.5) (width 0.5) (layer B.Cu) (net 20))
 (segment (start 38.5 115.5) (end 38.5 68.5) (width 0.5) (layer B.Cu) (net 20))
 (segment (start 48.58 58.42) (end 48.58 40) (width 0.5) (layer B.Cu) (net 20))
 (segment (start 38.5 68.5) (end 48.58 58.42) (width 0.5) (layer B.Cu) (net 20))
 (segment (start 24.08 141.11) (end 24.08 128.42) (width 0.5) (layer B.Cu) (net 21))
 (segment (start 24.08 128.42) (end 37.5 115) (width 0.5) (layer B.Cu) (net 21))
 (segment (start 37.5 115) (end 37.5 68) (width 0.5) (layer B.Cu) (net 21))
 (segment (start 47.56 57.94) (end 47.56 41) (width 0.5) (layer B.Cu) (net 21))
 (segment (start 37.5 68) (end 47.56 57.94) (width 0.5) (layer B.Cu) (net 21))
 (segment (start 22.81 143.65) (end 22.81 128.19) (width 0.5) (layer B.Cu) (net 22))
 (segment (start 22.81 128.19) (end 36.5 114.5) (width 0.5) (layer B.Cu) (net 22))
 (segment (start 36.5 114.5) (end 36.5 67.5) (width 0.5) (layer B.Cu) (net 22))
 (segment (start 46.54 57.46) (end 46.54 40) (width 0.5) (layer B.Cu) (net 22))
 (segment (start 36.5 67.5) (end 46.54 57.46) (width 0.5) (layer B.Cu) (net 22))
 (segment (start 21.54 141.11) (end 21.54 127.96) (width 0.5) (layer B.Cu) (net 23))
 (segment (start 21.54 127.96) (end 35.5 114) (width 0.5) (layer B.Cu) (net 23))
 (segment (start 35.5 114) (end 35.5 67) (width 0.5) (layer B.Cu) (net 23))
 (segment (start 45.52 56.98) (end 45.52 41) (width 0.5) (layer B.Cu) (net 23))
 (segment (start 35.5 67) (end 45.52 56.98) (width 0.5) (layer B.Cu) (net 23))
 (segment (start 20.27 143.65) (end 20.27 127.73) (width 0.5) (layer B.Cu) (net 24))
 (segment (start 20.27 127.73) (end 34.5 113.5) (width 0.5) (layer B.Cu) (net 24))
 (segment (start 34.5 113.5) (end 34.5 66.5) (width 0.5) (layer B.Cu) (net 24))
 (segment (start 34.5 66.5) (end 44.5 56.5) (width 0.5) (layer B.Cu) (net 24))
 (segment (start 44.5 56.5) (end 44.5 40) (width 0.5) (layer B.Cu) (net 24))
 (segment (start 31.49 187.68) (end 31.49 182.99) (width 2) (layer F.Cu) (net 34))
 (segment (start 31.49 182.99) (end 29.5 181) (width 2) (layer F.Cu) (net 34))
 (segment (start 29.5 181) (end 21 181) (width 2) (layer F.Cu) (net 34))
 (segment (start 21 181) (end 14.5 174.5) (width 2) (layer F.Cu) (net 34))
 (segment (start 15 30.5) (end 14.5 31) (width 1) (layer F.Cu) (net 34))
 (segment (start 23.5 30.5) (end 15 30.5) (width 1) (layer F.Cu) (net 34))
 (segment (start 14.5 31) (end 14.5 29) (width 2) (layer F.Cu) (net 34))
 (segment (start 15.5 60.5) (end 14.5 61.5) (width 1) (layer F.Cu) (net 34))
 (segment (start 23.5 60.5) (end 15.5 60.5) (width 1) (layer F.Cu) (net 34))
 (segment (start 14.5 61.5) (end 14.5 31) (width 2) (layer F.Cu) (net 34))
 (segment (start 23.5 90.5) (end 14.5 90.5) (width 1) (layer F.Cu) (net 34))
 (segment (start 14.5 90.5) (end 14.5 61.5) (width 2) (layer F.Cu) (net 34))
 (segment (start 15 120.5) (end 14.5 121) (width 1) (layer F.Cu) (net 34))
 (segment (start 23.5 120.5) (end 15 120.5) (width 1) (layer F.Cu) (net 34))
 (segment (start 14.5 174.5) (end 14.5 121) (width 2) (layer F.Cu) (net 34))
 (segment (start 14.5 121) (end 14.5 90.5) (width 2) (layer F.Cu) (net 34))
 (segment (start 24 187.68) (end 24 184) (width 2) (layer F.Cu) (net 33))
 (segment (start 24 184) (end 14.5 174.5) (width 2) (layer B.Cu) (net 33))
 (segment (start 14.5 31) (end 14.5 29) (width 2) (layer B.Cu) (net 33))
 (segment (start 14.7 118.7) (end 14.5 118.5) (width 1) (layer B.Cu) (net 33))
 (segment (start 23.5 118.7) (end 14.7 118.7) (width 1) (layer B.Cu) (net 33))
 (segment (start 14.5 174.5) (end 14.5 118.5) (width 2) (layer B.Cu) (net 33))
 (segment (start 14.7 88.7) (end 14.5 88.5) (width 1) (layer B.Cu) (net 33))
 (segment (start 23.5 88.7) (end 14.7 88.7) (width 1) (layer B.Cu) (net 33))
 (segment (start 14.5 118.5) (end 14.5 88.5) (width 2) (layer B.Cu) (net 33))
 (segment (start 14.8 58.7) (end 14.5 59) (width 1) (layer B.Cu) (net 33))
 (segment (start 14.5 88.5) (end 14.5 59) (width 2) (layer B.Cu) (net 33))
 (segment (start 23.5 58.7) (end 14.8 58.7) (width 1) (layer B.Cu) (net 33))
 (segment (start 14.5 59) (end 14.5 31) (width 2) (layer B.Cu) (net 33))
 (segment (start 14.8 28.7) (end 14.5 29) (width 1) (layer B.Cu) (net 33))
 (segment (start 23.5 28.7) (end 14.8 28.7) (width 1) (layer B.Cu) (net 33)))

